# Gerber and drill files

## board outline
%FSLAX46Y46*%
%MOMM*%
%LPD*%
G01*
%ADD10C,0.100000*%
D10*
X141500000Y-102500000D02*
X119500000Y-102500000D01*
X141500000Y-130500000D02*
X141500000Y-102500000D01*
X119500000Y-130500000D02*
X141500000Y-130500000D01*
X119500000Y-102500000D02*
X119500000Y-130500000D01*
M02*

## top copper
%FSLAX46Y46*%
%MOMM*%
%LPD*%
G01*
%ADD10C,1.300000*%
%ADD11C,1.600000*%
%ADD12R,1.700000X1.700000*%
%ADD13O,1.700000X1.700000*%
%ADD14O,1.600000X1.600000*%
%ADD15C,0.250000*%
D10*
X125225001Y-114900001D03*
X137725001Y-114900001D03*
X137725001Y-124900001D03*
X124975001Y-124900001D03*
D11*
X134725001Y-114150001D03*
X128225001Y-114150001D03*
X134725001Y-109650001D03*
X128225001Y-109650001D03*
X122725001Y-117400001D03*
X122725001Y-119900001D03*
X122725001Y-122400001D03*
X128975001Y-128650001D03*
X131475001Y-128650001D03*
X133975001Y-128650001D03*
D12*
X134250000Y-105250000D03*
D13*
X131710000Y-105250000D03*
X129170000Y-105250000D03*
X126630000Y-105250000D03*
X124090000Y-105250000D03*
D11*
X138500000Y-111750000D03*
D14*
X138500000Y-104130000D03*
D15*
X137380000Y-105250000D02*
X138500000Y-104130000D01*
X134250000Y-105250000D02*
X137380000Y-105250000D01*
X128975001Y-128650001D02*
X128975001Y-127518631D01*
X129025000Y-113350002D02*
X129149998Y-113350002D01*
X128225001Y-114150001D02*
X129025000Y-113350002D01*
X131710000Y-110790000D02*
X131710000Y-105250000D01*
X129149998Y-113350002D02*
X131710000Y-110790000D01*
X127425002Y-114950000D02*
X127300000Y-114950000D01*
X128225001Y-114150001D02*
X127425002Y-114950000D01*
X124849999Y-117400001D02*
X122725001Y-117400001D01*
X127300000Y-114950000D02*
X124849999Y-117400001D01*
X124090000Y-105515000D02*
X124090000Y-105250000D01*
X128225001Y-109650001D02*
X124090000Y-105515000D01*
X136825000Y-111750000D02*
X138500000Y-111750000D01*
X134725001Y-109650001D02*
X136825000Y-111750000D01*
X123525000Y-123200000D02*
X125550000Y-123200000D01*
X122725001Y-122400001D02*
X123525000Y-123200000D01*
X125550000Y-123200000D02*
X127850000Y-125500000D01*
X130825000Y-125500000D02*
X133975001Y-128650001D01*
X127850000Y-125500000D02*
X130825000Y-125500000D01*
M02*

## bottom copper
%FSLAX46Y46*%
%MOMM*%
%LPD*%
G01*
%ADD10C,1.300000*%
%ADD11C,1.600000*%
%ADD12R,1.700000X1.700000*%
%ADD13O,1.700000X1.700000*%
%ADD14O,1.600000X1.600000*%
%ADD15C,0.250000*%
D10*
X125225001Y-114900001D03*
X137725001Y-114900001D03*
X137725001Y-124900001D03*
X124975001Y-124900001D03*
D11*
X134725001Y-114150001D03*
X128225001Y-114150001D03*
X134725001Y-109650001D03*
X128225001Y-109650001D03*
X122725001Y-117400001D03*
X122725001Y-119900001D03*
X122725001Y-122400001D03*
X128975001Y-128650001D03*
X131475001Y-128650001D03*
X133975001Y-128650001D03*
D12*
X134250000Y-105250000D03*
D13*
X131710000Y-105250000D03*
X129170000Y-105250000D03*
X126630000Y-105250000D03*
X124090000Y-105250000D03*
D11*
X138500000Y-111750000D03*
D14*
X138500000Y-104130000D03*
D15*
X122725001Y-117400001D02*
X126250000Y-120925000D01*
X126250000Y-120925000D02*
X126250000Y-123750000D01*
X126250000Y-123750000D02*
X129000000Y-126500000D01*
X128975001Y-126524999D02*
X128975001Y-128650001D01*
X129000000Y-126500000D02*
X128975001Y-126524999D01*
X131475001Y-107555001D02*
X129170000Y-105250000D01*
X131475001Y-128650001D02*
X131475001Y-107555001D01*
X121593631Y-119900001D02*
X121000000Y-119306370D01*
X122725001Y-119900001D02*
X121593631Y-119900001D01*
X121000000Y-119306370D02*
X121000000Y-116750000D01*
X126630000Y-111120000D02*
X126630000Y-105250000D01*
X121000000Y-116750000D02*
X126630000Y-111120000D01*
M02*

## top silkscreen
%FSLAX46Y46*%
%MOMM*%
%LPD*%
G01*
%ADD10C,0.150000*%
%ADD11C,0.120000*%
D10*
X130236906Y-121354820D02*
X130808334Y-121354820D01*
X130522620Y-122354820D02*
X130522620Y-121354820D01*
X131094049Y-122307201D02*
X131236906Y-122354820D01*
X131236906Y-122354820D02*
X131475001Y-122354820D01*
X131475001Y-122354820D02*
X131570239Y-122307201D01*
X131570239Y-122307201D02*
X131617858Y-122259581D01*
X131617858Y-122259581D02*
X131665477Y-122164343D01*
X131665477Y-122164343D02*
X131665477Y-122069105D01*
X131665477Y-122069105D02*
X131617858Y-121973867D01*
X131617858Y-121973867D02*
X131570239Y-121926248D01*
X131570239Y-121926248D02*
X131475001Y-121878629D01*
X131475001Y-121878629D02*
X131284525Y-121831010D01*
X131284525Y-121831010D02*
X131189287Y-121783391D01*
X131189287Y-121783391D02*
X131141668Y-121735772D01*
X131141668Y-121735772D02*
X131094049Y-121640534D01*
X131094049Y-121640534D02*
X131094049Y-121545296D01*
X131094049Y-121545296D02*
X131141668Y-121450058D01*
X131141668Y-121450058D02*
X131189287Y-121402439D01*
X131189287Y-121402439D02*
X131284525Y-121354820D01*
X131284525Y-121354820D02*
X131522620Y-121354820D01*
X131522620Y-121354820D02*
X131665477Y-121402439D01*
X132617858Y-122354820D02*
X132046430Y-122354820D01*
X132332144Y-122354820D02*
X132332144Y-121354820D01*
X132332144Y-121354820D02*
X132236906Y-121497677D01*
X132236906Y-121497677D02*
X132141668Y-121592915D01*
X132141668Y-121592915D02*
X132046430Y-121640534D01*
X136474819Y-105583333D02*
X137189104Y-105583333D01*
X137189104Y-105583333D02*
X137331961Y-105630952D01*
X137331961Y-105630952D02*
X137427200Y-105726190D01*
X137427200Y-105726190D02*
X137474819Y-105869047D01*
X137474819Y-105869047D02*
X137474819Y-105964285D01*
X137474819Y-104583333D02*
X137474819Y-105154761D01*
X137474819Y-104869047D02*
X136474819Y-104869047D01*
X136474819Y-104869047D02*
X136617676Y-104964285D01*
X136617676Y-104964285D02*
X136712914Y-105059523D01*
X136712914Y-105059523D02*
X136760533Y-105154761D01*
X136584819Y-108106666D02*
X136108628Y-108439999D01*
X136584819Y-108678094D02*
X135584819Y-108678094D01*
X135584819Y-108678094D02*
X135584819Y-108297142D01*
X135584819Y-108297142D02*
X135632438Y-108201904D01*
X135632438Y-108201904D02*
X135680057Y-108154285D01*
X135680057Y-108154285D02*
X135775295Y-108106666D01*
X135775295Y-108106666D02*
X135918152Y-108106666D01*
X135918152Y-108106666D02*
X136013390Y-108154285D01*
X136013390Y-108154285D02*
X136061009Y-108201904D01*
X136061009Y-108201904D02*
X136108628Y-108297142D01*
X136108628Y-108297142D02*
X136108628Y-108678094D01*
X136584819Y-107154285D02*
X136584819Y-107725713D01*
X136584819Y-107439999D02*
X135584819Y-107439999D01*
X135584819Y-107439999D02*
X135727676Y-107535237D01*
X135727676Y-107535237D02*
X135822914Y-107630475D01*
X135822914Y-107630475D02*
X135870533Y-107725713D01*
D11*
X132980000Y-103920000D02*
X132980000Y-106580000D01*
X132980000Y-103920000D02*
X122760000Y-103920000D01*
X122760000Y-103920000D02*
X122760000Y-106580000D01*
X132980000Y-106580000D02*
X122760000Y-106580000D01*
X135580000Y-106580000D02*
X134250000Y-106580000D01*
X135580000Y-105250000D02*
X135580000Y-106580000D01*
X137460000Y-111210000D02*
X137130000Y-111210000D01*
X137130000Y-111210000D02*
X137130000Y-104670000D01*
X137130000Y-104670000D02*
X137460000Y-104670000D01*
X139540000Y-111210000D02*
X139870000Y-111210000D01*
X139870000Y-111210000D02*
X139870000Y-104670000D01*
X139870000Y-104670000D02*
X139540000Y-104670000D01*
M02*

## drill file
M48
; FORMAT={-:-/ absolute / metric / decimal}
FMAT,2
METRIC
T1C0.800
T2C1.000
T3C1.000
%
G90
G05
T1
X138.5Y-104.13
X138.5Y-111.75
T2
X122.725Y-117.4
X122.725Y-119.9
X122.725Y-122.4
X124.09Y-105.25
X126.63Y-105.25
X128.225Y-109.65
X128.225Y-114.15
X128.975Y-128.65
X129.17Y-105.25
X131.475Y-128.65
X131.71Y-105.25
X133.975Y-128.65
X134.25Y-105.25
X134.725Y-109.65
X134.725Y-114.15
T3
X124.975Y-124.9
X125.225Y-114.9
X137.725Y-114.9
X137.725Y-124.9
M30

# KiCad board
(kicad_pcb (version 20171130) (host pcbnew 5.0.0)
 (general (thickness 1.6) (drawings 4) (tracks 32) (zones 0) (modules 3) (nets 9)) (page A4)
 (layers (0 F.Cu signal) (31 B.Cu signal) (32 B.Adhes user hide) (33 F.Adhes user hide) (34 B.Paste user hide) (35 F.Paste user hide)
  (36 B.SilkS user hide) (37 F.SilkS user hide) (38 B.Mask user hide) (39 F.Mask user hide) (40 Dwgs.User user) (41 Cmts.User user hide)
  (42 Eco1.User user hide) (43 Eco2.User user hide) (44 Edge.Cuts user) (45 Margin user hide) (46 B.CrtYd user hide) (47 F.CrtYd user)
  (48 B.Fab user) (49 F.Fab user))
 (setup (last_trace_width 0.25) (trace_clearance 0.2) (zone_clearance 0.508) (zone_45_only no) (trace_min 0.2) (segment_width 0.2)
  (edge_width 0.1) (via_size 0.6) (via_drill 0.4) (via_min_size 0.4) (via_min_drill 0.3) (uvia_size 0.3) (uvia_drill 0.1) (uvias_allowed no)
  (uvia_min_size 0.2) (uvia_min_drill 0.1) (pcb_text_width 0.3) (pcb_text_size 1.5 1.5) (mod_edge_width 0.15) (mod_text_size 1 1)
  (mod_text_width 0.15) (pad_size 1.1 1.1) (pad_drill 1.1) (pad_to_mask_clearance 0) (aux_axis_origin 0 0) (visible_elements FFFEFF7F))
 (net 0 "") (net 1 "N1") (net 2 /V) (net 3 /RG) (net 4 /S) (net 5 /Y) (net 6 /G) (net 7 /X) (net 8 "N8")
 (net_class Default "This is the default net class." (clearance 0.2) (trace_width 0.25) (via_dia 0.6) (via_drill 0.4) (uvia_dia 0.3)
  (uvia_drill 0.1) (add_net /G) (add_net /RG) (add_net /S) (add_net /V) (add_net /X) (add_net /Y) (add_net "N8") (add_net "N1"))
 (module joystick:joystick (layer F.Cu) (at 131.475001 119.900001)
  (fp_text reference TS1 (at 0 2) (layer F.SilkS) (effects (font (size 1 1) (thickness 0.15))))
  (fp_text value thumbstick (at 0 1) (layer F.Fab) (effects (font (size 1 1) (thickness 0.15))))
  (pad "" np_thru_hole circle (at -6.25 -5) (size 1.3 1.3) (drill 1) (layers *.Cu *.Mask))
  (pad "" np_thru_hole circle (at 6.25 -5) (size 1.3 1.3) (drill 1) (layers *.Cu *.Mask))
  (pad "" np_thru_hole circle (at 6.25 5) (size 1.3 1.3) (drill 1) (layers *.Cu *.Mask))
  (pad "" np_thru_hole circle (at -6.5 5) (size 1.3 1.3) (drill 1) (layers *.Cu *.Mask))
  (pad J4 thru_hole circle (at 3.25 -5.75) (size 1.6 1.6) (drill 1) (layers *.Cu *.Mask) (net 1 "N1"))
  (pad J3 thru_hole circle (at -3.25 -5.75) (size 1.6 1.6) (drill 1) (layers *.Cu *.Mask) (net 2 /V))
  (pad J2 thru_hole circle (at 3.25 -10.25) (size 1.6 1.6) (drill 1) (layers *.Cu *.Mask) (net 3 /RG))
  (pad J1 thru_hole circle (at -3.25 -10.25) (size 1.6 1.6) (drill 1) (layers *.Cu *.Mask) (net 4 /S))
  (pad YV thru_hole circle (at -8.75 -2.5) (size 1.6 1.6) (drill 1) (layers *.Cu *.Mask) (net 2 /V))
  (pad Y thru_hole circle (at -8.75 0) (size 1.6 1.6) (drill 1) (layers *.Cu *.Mask) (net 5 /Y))
  (pad YG thru_hole circle (at -8.75 2.5) (size 1.6 1.6) (drill 1) (layers *.Cu *.Mask) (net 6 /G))
  (pad XV thru_hole circle (at -2.5 8.75) (size 1.6 1.6) (drill 1) (layers *.Cu *.Mask) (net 2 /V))
  (pad X thru_hole circle (at 0 8.75) (size 1.6 1.6) (drill 1) (layers *.Cu *.Mask) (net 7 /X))
  (pad XG thru_hole circle (at 2.5 8.75) (size 1.6 1.6) (drill 1) (layers *.Cu *.Mask) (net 6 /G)))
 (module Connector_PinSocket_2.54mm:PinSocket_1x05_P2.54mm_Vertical (layer F.Cu) (at 134.25 105.25 270)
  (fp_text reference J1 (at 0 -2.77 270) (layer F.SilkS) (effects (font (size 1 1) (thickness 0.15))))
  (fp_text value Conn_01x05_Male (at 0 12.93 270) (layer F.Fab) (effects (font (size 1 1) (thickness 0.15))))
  (fp_line (start -1.33 1.27) (end 1.33 1.27) (layer F.SilkS) (width 0.12))
  (fp_line (start -1.33 1.27) (end -1.33 11.49) (layer F.SilkS) (width 0.12))
  (fp_line (start -1.33 11.49) (end 1.33 11.49) (layer F.SilkS) (width 0.12))
  (fp_line (start 1.33 1.27) (end 1.33 11.49) (layer F.SilkS) (width 0.12))
  (fp_line (start 1.33 -1.33) (end 1.33 0) (layer F.SilkS) (width 0.12))
  (fp_line (start 0 -1.33) (end 1.33 -1.33) (layer F.SilkS) (width 0.12))
  (pad 1 thru_hole rect (at 0 0 270) (size 1.7 1.7) (drill 1) (layers *.Cu *.Mask) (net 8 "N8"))
  (pad 2 thru_hole oval (at 0 2.54 270) (size 1.7 1.7) (drill 1) (layers *.Cu *.Mask) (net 2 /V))
  (pad 3 thru_hole oval (at 0 5.08 270) (size 1.7 1.7) (drill 1) (layers *.Cu *.Mask) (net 7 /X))
  (pad 4 thru_hole oval (at 0 7.62 270) (size 1.7 1.7) (drill 1) (layers *.Cu *.Mask) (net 5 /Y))
  (pad 5 thru_hole oval (at 0 10.16 270) (size 1.7 1.7) (drill 1) (layers *.Cu *.Mask) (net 4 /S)))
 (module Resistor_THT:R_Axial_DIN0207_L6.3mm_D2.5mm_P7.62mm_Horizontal (layer F.Cu) (at 138.5 111.75 90)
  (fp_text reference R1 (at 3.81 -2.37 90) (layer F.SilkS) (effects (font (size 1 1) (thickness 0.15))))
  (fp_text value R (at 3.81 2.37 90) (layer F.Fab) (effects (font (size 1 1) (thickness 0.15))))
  (fp_line (start 0.54 -1.04) (end 0.54 -1.37) (layer F.SilkS) (width 0.12))
  (fp_line (start 0.54 -1.37) (end 7.08 -1.37) (layer F.SilkS) (width 0.12))
  (fp_line (start 7.08 -1.37) (end 7.08 -1.04) (layer F.SilkS) (width 0.12))
  (fp_line (start 0.54 1.04) (end 0.54 1.37) (layer F.SilkS) (width 0.12))
  (fp_line (start 0.54 1.37) (end 7.08 1.37) (layer F.SilkS) (width 0.12))
  (fp_line (start 7.08 1.37) (end 7.08 1.04) (layer F.SilkS) (width 0.12))
  (pad 1 thru_hole circle (at 0 0 90) (size 1.6 1.6) (drill 0.8) (layers *.Cu *.Mask) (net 3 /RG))
  (pad 2 thru_hole oval (at 7.62 0 90) (size 1.6 1.6) (drill 0.8) (layers *.Cu *.Mask) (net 8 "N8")))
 (gr_line (start 141.5 102.5) (end 119.5 102.5) (layer Edge.Cuts) (width 0.1))
 (gr_line (start 141.5 130.5) (end 141.5 102.5) (layer Edge.Cuts) (width 0.1))
 (gr_line (start 119.5 130.5) (end 141.5 130.5) (layer Edge.Cuts) (width 0.1))
 (gr_line (start 119.5 102.5) (end 119.5 130.5) (layer Edge.Cuts) (width 0.1))
 (segment (start 137.38 105.25) (end 138.5 104.13) (width 0.25) (layer F.Cu) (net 8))
 (segment (start 134.25 105.25) (end 137.38 105.25) (width 0.25) (layer F.Cu) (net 8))
 (segment (start 128.975001 128.650001) (end 128.975001 127.518631) (width 0.25) (layer F.Cu) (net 2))
 (segment (start 129.025 113.350002) (end 129.149998 113.350002) (width 0.25) (layer F.Cu) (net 2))
 (segment (start 128.225001 114.150001) (end 129.025 113.350002) (width 0.25) (layer F.Cu) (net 2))
 (segment (start 131.71 110.79) (end 131.71 105.25) (width 0.25) (layer F.Cu) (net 2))
 (segment (start 129.149998 113.350002) (end 131.71 110.79) (width 0.25) (layer F.Cu) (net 2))
 (segment (start 127.425002 114.95) (end 127.3 114.95) (width 0.25) (layer F.Cu) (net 2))
 (segment (start 128.225001 114.150001) (end 127.425002 114.95) (width 0.25) (layer F.Cu) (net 2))
 (segment (start 124.849999 117.400001) (end 122.725001 117.400001) (width 0.25) (layer F.Cu) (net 2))
 (segment (start 127.3 114.95) (end 124.849999 117.400001) (width 0.25) (layer F.Cu) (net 2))
 (segment (start 122.725001 117.400001) (end 126.25 120.925) (width 0.25) (layer B.Cu) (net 2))
 (segment (start 126.25 120.925) (end 126.25 123.75) (width 0.25) (layer B.Cu) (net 2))
 (segment (start 126.25 123.75) (end 129 126.5) (width 0.25) (layer B.Cu) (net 2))
 (segment (start 128.975001 126.524999) (end 128.975001 128.650001) (width 0.25) (layer B.Cu) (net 2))
 (segment (start 129 126.5) (end 128.975001 126.524999) (width 0.25) (layer B.Cu) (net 2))
 (segment (start 131.475001 107.555001) (end 129.17 105.25) (width 0.25) (layer B.Cu) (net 7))
 (segment (start 131.475001 128.650001) (end 131.475001 107.555001) (width 0.25) (layer B.Cu) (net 7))
 (segment (start 121.593631 119.900001) (end 121 119.30637) (width 0.25) (layer B.Cu) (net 5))
 (segment (start 122.725001 119.900001) (end 121.593631 119.900001) (width 0.25) (layer B.Cu) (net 5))
 (segment (start 121 119.30637) (end 121 116.75) (width 0.25) (layer B.Cu) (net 5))
 (segment (start 126.63 111.12) (end 126.63 105.25) (width 0.25) (layer B.Cu) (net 5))
 (segment (start 121 116.75) (end 126.63 111.12) (width 0.25) (layer B.Cu) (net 5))
 (segment (start 124.09 105.515) (end 124.09 105.25) (width 0.25) (layer F.Cu) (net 4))
 (segment (start 128.225001 109.650001) (end 124.09 105.515) (width 0.25) (layer F.Cu) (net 4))
 (segment (start 136.825 111.75) (end 138.5 111.75) (width 0.25) (layer F.Cu) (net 3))
 (segment (start 134.725001 109.650001) (end 136.825 111.75) (width 0.25) (layer F.Cu) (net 3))
 (segment (start 123.525 123.2) (end 125.55 123.2) (width 0.25) (layer F.Cu) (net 6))
 (segment (start 122.725001 122.400001) (end 123.525 123.2) (width 0.25) (layer F.Cu) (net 6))
 (segment (start 125.55 123.2) (end 127.85 125.5) (width 0.25) (layer F.Cu) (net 6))
 (segment (start 130.825 125.5) (end 133.975001 128.650001) (width 0.25) (layer F.Cu) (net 6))
 (segment (start 127.85 125.5) (end 130.825 125.5) (width 0.25) (layer F.Cu) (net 6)))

